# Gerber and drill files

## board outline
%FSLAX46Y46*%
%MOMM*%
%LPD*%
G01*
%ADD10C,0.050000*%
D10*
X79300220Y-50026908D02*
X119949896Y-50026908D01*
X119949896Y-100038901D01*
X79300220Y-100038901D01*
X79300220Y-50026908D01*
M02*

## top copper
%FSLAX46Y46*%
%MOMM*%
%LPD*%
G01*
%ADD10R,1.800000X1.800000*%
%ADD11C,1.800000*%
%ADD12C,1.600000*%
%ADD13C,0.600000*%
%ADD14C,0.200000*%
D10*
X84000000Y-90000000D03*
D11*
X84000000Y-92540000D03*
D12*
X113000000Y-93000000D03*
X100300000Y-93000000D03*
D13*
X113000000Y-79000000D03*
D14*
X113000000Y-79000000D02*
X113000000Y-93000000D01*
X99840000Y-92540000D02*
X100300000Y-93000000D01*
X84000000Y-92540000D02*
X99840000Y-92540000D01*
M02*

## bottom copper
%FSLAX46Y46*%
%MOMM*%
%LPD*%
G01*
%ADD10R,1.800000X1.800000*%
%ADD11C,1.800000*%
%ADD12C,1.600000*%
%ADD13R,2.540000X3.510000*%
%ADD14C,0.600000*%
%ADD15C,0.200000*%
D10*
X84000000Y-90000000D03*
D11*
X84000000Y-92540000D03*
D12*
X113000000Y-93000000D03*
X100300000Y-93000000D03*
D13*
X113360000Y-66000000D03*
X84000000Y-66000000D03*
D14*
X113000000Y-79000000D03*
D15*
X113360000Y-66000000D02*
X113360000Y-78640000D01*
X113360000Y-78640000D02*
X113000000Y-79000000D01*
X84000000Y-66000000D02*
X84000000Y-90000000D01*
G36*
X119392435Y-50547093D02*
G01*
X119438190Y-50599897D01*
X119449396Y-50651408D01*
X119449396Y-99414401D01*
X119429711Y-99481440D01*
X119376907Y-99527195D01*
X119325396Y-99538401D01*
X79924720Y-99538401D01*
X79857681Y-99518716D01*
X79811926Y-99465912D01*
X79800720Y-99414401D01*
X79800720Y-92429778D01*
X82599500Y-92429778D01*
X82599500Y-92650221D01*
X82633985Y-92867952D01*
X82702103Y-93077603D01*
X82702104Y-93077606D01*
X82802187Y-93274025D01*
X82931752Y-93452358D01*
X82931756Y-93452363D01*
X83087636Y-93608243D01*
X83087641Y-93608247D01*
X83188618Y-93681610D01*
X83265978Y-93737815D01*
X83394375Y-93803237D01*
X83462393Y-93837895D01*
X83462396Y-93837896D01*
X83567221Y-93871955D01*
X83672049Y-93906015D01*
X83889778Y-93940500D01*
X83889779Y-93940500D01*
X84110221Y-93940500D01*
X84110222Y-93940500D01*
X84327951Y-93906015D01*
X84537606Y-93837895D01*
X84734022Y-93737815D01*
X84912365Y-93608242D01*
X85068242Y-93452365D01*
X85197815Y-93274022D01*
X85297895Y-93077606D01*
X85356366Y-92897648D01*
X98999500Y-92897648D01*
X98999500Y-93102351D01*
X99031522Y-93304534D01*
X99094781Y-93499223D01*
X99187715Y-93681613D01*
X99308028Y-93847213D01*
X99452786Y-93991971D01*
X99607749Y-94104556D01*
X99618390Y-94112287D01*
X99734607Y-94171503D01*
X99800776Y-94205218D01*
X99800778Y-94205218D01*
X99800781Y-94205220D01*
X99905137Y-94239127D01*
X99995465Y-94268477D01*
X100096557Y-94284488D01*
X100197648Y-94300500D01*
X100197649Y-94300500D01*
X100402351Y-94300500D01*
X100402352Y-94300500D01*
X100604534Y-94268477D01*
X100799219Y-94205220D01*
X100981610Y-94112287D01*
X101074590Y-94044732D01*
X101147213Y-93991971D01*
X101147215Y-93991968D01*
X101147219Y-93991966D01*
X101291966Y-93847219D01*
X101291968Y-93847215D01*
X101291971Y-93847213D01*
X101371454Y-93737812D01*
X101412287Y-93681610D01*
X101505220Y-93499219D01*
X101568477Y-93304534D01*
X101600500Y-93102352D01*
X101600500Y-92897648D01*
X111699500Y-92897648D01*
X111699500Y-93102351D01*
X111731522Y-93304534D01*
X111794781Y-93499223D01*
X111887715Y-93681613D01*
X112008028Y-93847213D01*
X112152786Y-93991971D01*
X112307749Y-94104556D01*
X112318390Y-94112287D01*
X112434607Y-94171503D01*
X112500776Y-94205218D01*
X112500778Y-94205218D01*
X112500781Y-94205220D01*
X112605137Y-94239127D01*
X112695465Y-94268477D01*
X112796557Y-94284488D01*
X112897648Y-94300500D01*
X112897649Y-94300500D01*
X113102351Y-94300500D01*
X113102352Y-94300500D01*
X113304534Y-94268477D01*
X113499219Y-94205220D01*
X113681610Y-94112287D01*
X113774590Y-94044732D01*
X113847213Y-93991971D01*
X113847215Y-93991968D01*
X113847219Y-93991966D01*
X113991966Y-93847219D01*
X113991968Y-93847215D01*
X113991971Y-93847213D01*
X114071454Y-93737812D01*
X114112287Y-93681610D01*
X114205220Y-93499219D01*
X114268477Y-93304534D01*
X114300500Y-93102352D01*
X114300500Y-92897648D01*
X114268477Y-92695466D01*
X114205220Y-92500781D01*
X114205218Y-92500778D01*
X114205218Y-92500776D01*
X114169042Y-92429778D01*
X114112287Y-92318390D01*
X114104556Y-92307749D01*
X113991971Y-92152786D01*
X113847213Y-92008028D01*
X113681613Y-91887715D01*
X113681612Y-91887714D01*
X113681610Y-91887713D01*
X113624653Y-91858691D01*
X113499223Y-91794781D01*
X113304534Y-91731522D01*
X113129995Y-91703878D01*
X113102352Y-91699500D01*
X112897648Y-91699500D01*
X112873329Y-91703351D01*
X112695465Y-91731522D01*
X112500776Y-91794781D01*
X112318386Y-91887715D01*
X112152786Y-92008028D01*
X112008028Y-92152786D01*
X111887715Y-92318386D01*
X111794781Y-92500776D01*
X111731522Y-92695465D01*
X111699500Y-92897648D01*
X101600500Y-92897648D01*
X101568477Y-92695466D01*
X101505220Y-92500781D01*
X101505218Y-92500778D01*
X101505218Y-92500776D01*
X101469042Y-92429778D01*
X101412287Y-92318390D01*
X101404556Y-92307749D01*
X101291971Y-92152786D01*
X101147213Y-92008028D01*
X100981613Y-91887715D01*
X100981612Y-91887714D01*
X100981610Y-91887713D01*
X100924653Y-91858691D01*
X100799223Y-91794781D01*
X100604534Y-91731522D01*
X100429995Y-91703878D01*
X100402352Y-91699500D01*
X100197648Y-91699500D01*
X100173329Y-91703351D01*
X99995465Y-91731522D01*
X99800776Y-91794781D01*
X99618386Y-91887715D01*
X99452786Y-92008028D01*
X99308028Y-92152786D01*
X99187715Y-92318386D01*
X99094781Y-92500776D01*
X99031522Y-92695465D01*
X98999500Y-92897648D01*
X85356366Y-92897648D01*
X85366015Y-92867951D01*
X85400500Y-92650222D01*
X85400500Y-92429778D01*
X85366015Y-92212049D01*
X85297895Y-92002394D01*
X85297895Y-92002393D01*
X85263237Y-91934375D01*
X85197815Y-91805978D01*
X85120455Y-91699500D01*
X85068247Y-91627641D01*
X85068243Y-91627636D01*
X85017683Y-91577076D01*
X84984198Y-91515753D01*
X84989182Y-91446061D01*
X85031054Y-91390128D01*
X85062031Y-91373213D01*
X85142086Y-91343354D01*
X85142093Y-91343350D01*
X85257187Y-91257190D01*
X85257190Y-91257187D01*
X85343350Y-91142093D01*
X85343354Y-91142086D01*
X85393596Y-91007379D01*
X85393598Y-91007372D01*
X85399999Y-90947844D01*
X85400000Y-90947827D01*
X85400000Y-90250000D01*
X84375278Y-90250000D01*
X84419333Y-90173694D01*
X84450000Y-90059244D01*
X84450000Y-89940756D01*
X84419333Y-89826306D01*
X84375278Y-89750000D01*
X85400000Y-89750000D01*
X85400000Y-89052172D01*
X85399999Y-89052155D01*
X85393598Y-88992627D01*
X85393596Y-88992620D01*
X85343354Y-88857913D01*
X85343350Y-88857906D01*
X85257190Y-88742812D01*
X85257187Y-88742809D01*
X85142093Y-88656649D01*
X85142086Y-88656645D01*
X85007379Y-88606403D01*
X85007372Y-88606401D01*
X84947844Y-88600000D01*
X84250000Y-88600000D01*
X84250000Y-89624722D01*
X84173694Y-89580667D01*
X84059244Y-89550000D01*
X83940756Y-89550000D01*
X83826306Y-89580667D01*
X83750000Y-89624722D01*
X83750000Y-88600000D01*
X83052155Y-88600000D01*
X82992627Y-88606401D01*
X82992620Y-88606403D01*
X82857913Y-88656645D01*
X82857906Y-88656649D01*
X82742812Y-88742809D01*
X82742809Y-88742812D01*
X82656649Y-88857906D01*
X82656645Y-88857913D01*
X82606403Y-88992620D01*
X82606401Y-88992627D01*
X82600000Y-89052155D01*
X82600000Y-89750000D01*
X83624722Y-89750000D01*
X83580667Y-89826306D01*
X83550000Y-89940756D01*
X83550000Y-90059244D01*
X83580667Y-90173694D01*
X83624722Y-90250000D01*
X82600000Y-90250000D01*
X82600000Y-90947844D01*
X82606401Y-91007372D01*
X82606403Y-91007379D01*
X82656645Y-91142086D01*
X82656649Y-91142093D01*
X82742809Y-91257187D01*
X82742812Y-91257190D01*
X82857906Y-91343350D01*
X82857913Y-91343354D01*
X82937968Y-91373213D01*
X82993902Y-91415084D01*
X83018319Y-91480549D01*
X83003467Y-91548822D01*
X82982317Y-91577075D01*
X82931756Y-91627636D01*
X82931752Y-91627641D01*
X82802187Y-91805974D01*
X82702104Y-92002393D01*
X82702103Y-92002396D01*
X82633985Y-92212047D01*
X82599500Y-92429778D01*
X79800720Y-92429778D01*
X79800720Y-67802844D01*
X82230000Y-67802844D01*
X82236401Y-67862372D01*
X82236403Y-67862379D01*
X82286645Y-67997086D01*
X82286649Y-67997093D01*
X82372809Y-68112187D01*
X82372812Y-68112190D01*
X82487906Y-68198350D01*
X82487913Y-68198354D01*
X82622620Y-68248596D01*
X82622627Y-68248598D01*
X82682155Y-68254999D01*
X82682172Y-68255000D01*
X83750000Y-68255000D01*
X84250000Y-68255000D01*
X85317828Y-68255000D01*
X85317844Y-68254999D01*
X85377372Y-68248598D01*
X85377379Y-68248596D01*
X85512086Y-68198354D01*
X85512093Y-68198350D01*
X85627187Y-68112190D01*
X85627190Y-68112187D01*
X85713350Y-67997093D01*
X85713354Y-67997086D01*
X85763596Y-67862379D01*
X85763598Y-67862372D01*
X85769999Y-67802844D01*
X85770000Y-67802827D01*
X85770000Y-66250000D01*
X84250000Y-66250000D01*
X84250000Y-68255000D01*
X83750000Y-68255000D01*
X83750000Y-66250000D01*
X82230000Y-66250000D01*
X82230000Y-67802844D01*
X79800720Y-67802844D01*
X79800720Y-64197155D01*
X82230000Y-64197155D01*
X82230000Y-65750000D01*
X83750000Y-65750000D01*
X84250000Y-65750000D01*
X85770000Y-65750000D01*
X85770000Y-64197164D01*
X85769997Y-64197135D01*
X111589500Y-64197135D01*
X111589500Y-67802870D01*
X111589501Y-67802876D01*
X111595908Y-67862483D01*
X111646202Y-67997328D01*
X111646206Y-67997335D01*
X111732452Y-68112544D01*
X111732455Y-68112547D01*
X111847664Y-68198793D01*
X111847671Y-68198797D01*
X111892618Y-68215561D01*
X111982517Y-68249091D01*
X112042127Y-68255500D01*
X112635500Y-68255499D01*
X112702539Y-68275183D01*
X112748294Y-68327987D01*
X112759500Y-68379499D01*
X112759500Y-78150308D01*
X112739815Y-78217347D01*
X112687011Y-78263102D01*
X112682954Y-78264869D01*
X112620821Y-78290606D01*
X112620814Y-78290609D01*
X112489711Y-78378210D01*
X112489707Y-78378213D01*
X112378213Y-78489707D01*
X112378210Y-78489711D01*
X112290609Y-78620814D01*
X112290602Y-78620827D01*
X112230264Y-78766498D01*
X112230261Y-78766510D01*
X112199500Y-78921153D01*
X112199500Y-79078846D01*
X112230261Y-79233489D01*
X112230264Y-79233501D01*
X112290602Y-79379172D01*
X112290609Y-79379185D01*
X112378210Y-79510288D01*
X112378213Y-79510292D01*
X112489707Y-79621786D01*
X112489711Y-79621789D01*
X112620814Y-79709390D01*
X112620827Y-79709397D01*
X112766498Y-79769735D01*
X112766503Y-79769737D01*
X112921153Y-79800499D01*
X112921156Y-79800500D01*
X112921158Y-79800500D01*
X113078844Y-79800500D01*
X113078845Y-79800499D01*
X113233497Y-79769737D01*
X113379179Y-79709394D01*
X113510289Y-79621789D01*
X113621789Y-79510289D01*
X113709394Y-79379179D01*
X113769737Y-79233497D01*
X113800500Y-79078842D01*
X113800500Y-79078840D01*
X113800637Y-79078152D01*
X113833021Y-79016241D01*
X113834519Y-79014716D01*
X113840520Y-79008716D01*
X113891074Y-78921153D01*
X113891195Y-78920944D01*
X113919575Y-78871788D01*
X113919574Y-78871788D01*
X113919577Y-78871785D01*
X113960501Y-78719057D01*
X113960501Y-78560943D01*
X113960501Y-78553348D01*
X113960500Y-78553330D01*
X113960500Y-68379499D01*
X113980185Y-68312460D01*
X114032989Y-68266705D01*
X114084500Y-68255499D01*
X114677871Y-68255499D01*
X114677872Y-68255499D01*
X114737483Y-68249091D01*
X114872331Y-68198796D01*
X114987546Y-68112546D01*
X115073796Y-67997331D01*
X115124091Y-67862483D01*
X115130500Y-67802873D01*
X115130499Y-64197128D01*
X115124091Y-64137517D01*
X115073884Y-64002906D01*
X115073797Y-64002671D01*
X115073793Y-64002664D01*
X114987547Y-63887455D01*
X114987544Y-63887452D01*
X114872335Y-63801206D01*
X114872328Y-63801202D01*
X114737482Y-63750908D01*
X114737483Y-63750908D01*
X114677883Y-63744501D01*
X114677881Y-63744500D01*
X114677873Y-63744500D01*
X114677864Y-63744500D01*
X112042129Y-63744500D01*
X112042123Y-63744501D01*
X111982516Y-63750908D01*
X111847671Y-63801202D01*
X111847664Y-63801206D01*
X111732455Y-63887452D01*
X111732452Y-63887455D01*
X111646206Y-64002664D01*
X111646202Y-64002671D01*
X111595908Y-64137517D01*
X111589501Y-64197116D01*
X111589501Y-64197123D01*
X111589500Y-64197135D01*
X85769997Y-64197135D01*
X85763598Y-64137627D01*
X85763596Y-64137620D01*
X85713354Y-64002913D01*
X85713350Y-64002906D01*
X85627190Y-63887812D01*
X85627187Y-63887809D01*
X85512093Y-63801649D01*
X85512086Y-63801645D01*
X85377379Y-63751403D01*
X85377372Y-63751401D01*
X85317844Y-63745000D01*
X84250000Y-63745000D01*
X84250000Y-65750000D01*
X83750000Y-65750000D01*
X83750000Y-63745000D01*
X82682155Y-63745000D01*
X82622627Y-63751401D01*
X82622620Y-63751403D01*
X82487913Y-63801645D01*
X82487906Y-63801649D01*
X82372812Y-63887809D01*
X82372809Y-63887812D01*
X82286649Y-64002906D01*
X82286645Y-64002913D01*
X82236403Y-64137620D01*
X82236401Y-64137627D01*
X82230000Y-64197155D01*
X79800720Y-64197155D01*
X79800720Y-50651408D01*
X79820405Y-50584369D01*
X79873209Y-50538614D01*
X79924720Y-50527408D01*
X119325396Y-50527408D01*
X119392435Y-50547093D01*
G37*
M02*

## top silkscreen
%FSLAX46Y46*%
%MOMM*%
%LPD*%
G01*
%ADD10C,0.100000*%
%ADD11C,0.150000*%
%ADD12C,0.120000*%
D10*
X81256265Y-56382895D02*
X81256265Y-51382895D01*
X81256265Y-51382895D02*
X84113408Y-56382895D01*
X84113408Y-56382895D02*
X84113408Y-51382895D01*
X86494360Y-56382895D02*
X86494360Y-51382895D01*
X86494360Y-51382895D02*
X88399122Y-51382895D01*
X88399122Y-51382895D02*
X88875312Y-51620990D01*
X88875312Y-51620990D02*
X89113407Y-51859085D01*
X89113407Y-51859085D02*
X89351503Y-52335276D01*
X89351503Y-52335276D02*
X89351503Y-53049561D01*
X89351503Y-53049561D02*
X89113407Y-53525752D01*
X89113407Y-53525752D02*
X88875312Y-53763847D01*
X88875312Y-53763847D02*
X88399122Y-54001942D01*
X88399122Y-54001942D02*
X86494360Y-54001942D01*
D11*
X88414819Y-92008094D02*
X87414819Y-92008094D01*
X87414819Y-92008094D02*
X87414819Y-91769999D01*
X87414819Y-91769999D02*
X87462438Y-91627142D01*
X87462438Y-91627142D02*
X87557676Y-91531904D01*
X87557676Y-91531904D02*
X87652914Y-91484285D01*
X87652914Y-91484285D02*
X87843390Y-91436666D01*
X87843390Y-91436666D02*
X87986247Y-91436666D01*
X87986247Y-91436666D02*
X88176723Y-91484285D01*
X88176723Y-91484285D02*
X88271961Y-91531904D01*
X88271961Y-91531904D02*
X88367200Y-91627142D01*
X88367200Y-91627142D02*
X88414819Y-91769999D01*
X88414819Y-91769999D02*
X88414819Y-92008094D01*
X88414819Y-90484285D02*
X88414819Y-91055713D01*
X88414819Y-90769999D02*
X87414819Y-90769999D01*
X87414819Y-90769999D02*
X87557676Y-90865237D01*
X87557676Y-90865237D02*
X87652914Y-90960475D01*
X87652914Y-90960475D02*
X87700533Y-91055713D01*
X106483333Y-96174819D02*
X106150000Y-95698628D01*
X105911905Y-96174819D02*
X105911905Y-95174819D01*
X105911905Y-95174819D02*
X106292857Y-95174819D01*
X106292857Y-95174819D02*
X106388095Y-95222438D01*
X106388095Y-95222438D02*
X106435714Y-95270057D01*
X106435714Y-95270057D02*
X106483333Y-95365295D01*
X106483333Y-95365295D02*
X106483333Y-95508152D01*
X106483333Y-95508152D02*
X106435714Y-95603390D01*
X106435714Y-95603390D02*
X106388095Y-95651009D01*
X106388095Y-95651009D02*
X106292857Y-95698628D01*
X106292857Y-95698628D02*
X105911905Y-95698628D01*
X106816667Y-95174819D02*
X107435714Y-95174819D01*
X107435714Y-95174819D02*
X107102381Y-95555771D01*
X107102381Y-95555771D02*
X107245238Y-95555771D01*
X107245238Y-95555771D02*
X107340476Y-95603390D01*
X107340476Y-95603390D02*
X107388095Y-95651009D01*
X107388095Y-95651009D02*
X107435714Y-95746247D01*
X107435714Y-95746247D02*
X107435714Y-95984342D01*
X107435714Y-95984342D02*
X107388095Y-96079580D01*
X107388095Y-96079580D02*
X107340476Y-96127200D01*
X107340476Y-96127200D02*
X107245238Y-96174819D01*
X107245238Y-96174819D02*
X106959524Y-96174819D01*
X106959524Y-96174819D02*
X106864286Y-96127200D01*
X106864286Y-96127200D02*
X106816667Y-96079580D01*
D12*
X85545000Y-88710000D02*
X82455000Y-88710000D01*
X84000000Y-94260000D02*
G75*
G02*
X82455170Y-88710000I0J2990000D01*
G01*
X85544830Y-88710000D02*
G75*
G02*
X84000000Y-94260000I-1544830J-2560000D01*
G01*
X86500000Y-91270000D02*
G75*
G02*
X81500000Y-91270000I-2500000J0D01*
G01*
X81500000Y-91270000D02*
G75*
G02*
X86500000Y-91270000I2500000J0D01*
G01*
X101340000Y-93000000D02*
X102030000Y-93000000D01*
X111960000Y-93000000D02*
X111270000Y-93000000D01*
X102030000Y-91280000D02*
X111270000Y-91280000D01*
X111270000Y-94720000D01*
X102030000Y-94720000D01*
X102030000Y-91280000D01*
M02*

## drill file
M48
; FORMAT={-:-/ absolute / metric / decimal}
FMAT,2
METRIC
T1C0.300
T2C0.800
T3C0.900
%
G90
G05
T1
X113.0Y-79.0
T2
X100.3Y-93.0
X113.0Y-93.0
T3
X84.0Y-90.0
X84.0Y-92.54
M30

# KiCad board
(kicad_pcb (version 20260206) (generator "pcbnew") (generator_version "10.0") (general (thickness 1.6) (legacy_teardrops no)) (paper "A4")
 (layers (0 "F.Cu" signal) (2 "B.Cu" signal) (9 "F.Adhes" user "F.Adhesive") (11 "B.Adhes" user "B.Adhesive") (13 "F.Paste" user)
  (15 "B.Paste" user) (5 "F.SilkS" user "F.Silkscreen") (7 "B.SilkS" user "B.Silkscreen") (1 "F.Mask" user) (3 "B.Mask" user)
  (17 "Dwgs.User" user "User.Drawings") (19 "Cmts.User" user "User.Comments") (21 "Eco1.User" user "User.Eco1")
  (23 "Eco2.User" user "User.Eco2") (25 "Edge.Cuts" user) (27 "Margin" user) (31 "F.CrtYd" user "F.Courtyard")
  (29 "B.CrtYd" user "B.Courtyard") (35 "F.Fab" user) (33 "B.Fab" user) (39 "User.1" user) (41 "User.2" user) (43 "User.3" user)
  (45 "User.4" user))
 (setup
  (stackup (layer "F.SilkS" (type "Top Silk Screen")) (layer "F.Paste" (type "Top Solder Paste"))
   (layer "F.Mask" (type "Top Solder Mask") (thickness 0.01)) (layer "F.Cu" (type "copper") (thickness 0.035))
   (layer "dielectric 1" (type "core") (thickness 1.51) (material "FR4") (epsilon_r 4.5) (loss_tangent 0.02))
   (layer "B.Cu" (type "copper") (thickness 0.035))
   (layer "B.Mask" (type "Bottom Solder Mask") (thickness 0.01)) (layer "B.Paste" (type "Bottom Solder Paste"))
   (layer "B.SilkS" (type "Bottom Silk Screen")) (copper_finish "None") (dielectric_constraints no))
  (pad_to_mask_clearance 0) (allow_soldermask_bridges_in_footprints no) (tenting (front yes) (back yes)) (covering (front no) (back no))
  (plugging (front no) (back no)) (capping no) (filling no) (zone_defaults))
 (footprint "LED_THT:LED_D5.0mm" (layer "F.Cu") (at 84 90 -90)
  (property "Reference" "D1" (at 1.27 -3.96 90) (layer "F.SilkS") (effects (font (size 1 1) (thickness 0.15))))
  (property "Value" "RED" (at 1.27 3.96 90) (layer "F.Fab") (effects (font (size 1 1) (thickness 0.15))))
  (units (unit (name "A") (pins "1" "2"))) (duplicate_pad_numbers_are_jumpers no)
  (fp_line (start -1.29 -1.545) (end -1.29 1.545) (stroke (width 0.12) (type solid)) (layer "F.SilkS"))
  (fp_arc (start 4.26 0) (mid 2.071779 2.880495) (end -1.29 1.54483) (stroke (width 0.12) (type solid)) (layer "F.SilkS"))
  (fp_arc (start -1.29 -1.54483) (mid 2.071779 -2.880495) (end 4.26 0) (stroke (width 0.12) (type solid)) (layer "F.SilkS"))
  (fp_circle (center 1.27 0) (end 3.77 0) (stroke (width 0.12) (type solid)) (fill no) (layer "F.SilkS"))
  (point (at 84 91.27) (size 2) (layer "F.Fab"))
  (pad "1" thru_hole rect (at 0 0 270) (size 1.8 1.8) (drill 0.9) (layers "*.Cu" "*.Mask") (remove_unused_layers no) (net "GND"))
  (pad "2" thru_hole circle (at 2.54 0 270) (size 1.8 1.8) (drill 0.9) (layers "*.Cu" "*.Mask") (remove_unused_layers no) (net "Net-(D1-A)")))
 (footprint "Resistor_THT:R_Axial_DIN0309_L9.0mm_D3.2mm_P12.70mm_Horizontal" (layer "F.Cu") (at 113 93 180)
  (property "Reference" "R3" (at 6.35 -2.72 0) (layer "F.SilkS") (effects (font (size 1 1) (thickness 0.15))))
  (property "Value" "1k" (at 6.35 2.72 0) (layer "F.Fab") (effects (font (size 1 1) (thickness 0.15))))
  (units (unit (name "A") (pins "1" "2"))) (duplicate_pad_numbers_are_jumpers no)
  (fp_line (start 11.66 0) (end 10.97 0) (stroke (width 0.12) (type solid)) (layer "F.SilkS"))
  (fp_line (start 1.04 0) (end 1.73 0) (stroke (width 0.12) (type solid)) (layer "F.SilkS"))
  (fp_rect (start 1.73 -1.72) (end 10.97 1.72) (stroke (width 0.12) (type solid)) (fill no) (layer "F.SilkS"))
  (pad "1" thru_hole circle (at 0 0 180) (size 1.6 1.6) (drill 0.8) (layers "*.Cu" "*.Mask") (remove_unused_layers no) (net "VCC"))
  (pad "2" thru_hole circle (at 12.7 0 180) (size 1.6 1.6) (drill 0.8) (layers "*.Cu" "*.Mask") (remove_unused_layers no) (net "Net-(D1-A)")))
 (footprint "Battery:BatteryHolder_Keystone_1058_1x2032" (layer "B.Cu") (at 98.68 66 180)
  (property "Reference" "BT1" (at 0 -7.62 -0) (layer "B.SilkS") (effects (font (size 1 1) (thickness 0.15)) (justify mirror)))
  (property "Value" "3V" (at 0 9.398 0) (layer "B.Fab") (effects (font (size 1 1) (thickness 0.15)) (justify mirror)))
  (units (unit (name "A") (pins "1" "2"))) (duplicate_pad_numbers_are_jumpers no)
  (pad "1" smd rect (at -14.68 0 180) (size 2.54 3.51) (layers "B.Cu" "B.Mask" "B.Paste") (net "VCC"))
  (pad "2" smd rect (at 14.68 0 180) (size 2.54 3.51) (layers "B.Cu" "B.Mask" "B.Paste") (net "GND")))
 (gr_rect (start 79.30022 50.026908) (end 119.949896 100.038901) (stroke (width 0.05) (type default)) (fill no) (layer "Edge.Cuts"))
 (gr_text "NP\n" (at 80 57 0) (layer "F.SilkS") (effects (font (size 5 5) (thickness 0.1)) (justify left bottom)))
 (segment (start 113 79) (end 113 93) (width 0.2) (layer "F.Cu") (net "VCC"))
 (via (at 113 79) (size 0.6) (drill 0.3) (layers "F.Cu" "B.Cu") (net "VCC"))
 (segment (start 113.36 66) (end 113.36 78.64) (width 0.2) (layer "B.Cu") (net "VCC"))
 (segment (start 113.36 78.64) (end 113 79) (width 0.2) (layer "B.Cu") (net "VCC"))
 (segment (start 84 66) (end 84 90) (width 0.2) (layer "B.Cu") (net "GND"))
 (segment (start 99.84 92.54) (end 100.3 93) (width 0.2) (layer "F.Cu") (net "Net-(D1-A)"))
 (segment (start 84 92.54) (end 99.84 92.54) (width 0.2) (layer "F.Cu") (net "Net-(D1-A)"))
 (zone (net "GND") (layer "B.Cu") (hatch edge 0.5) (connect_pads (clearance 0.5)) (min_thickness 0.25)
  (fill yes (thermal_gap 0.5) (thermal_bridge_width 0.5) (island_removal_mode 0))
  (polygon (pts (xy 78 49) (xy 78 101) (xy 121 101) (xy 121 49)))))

